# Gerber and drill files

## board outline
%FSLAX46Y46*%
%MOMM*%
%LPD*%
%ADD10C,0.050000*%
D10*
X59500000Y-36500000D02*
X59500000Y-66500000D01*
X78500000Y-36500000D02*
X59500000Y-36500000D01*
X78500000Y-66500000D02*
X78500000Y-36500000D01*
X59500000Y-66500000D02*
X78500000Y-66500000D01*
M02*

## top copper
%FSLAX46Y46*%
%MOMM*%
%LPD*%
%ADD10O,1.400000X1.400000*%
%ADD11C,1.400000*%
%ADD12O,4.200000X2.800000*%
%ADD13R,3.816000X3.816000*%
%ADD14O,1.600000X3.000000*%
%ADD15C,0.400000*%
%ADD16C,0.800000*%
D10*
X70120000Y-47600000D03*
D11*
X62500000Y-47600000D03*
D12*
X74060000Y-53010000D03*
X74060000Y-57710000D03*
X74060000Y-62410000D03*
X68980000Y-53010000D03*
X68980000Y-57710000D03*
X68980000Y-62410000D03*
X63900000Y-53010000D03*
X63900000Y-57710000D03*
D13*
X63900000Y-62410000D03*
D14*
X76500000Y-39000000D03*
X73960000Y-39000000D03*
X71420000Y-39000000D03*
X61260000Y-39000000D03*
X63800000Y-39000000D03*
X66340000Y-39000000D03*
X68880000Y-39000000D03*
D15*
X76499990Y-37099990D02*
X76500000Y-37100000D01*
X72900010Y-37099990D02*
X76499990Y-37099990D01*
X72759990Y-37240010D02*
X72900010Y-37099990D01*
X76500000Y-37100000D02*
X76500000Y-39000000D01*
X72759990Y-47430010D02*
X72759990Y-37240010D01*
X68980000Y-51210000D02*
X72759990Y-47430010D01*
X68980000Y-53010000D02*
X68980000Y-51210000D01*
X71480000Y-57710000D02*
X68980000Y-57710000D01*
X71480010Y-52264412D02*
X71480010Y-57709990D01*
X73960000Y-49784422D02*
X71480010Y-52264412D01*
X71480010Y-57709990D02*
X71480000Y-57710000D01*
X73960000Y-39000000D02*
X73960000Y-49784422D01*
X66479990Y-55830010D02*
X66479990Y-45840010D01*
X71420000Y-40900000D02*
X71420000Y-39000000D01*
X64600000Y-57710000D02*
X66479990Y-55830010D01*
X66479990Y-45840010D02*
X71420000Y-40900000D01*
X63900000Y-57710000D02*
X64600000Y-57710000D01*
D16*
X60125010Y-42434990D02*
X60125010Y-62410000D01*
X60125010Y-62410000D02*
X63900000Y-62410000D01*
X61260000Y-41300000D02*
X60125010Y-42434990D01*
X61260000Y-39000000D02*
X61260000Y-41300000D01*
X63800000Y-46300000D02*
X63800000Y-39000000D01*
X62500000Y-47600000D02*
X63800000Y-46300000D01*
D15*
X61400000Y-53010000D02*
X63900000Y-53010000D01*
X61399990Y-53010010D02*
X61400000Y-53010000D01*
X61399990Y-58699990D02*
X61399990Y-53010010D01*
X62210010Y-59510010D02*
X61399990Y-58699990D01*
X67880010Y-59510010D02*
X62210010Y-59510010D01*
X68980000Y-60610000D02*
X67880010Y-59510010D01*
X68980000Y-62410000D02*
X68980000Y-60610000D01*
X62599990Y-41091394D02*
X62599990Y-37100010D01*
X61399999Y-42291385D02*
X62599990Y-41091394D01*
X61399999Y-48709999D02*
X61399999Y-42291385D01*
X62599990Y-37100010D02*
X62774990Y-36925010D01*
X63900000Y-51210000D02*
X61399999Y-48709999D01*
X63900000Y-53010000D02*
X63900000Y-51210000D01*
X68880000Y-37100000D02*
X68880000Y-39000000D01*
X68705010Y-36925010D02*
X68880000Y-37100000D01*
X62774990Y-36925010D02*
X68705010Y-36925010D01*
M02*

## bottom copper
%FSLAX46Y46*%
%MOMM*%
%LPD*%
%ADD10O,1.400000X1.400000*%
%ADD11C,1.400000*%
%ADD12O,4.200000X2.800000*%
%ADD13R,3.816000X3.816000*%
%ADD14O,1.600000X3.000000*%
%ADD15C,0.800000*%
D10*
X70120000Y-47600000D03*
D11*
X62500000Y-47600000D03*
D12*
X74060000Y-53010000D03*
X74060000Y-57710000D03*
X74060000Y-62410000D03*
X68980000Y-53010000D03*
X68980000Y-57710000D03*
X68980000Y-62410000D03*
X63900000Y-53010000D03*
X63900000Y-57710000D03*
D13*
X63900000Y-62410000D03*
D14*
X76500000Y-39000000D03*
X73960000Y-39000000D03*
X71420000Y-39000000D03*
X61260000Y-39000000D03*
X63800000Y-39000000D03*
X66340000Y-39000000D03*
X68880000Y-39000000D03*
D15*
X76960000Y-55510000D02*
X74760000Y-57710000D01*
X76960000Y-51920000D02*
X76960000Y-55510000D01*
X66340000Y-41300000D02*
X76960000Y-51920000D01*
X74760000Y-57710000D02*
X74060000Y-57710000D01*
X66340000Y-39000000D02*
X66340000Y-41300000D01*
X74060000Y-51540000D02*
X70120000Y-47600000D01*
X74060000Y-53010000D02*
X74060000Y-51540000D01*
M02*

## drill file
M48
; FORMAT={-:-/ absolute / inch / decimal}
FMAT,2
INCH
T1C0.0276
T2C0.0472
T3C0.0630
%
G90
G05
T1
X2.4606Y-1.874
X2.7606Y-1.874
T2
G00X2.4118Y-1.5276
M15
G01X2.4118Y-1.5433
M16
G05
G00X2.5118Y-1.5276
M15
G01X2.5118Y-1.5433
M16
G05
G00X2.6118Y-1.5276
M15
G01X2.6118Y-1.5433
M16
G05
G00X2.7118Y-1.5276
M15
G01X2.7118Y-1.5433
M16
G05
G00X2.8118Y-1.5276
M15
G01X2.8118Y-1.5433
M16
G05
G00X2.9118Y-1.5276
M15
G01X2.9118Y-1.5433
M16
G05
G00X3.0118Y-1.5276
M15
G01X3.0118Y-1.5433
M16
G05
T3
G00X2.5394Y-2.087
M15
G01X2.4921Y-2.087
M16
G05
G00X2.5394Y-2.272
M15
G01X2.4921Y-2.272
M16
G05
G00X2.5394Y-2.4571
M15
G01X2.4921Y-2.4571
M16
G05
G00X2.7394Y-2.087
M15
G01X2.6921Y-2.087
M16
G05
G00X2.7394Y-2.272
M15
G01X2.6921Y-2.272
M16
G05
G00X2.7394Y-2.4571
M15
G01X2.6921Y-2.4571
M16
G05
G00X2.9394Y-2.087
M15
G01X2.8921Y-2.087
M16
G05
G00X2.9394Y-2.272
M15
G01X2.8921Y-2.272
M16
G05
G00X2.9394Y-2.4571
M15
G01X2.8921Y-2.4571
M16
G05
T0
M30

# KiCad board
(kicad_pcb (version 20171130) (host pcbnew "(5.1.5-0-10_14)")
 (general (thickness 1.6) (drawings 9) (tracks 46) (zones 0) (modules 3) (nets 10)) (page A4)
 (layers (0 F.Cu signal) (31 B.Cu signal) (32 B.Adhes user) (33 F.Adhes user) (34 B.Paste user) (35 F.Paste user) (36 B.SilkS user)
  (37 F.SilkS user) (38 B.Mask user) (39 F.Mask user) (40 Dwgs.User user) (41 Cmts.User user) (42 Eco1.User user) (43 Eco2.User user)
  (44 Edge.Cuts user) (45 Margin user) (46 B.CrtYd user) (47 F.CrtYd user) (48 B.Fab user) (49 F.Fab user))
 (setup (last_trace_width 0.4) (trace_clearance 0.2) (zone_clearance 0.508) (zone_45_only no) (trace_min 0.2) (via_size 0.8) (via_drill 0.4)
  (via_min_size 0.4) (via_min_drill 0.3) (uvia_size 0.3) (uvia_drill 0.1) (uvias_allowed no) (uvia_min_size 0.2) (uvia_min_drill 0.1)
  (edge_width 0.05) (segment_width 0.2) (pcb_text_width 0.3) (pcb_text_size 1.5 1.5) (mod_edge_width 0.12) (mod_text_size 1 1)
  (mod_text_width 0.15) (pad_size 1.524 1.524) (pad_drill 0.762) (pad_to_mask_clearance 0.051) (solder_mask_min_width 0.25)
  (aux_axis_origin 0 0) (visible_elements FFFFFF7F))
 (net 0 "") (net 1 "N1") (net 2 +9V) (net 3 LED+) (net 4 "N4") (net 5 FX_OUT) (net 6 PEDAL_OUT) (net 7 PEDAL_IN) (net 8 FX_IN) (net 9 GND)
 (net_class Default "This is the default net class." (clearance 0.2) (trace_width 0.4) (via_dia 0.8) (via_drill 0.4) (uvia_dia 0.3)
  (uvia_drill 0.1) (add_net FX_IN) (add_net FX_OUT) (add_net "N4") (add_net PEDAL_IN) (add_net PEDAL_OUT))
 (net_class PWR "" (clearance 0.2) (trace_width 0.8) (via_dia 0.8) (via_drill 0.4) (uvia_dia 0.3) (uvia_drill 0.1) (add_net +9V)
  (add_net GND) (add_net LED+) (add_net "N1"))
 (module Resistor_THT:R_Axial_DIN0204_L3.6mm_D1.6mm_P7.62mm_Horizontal (layer B.Cu) (at 62.5 47.6)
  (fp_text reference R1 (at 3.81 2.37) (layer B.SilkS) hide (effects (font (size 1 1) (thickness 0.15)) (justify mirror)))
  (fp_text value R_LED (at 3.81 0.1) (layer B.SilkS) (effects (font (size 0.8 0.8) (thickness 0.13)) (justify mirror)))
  (pad 2 thru_hole oval (at 7.62 0) (size 1.4 1.4) (drill 0.7) (layers *.Cu *.Mask) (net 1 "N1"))
  (pad 1 thru_hole circle (at 0 0) (size 1.4 1.4) (drill 0.7) (layers *.Cu *.Mask) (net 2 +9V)))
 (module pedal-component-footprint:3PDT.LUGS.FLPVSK (layer B.Cu) (at 68.98 57.71)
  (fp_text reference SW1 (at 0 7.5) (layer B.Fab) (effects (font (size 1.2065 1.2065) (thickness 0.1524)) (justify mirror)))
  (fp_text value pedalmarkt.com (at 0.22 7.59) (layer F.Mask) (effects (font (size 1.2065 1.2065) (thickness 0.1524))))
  (pad 9 thru_hole oval (at 5.08 -4.7 180) (size 4.2 2.8) (drill oval 2.8 1.6) (layers *.Cu *.Mask) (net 1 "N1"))
  (pad 8 thru_hole oval (at 5.08 0 180) (size 4.2 2.8) (drill oval 2.8 1.6) (layers *.Cu *.Mask) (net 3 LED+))
  (pad 7 thru_hole oval (at 5.08 4.7 180) (size 4.2 2.8) (drill oval 2.8 1.6) (layers *.Cu *.Mask) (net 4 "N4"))
  (pad 6 thru_hole oval (at 0 -4.7 180) (size 4.2 2.8) (drill oval 2.8 1.6) (layers *.Cu *.Mask) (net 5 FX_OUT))
  (pad 5 thru_hole oval (at 0 0 180) (size 4.2 2.8) (drill oval 2.8 1.6) (layers *.Cu *.Mask) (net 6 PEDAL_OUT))
  (pad 4 thru_hole oval (at 0 4.7 180) (size 4.2 2.8) (drill oval 2.8 1.6) (layers *.Cu *.Mask) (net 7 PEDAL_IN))
  (pad 3 thru_hole oval (at -5.08 -4.7 180) (size 4.2 2.8) (drill oval 2.8 1.6) (layers *.Cu *.Mask) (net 7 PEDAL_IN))
  (pad 2 thru_hole oval (at -5.08 0 180) (size 4.2 2.8) (drill oval 2.8 1.6) (layers *.Cu *.Mask) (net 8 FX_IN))
  (pad 1 thru_hole rect (at -5.08 4.7 180) (size 3.816 3.816) (drill oval 2.8 1.6) (layers *.Cu *.Mask) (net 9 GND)))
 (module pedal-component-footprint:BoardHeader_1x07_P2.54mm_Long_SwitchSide (layer F.Cu) (at 68.88 39)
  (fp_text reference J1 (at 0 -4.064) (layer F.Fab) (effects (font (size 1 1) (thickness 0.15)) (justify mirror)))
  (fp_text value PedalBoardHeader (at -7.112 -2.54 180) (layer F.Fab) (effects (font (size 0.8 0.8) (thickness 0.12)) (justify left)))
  (pad 7 thru_hole oval (at 7.62 0) (size 1.6 3) (drill oval 1.2 1.6) (layers *.Cu *.Mask) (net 5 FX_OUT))
  (pad 6 thru_hole oval (at 5.08 0) (size 1.6 3) (drill oval 1.2 1.6) (layers *.Cu *.Mask) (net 6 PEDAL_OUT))
  (pad 5 thru_hole oval (at 2.54 0) (size 1.6 3) (drill oval 1.2 1.6) (layers *.Cu *.Mask) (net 8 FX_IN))
  (pad 1 thru_hole oval (at -7.62 0) (size 1.6 3) (drill oval 1.2 1.6) (layers *.Cu *.Mask) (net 9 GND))
  (pad 2 thru_hole oval (at -5.08 0) (size 1.6 3) (drill oval 1.2 1.6) (layers *.Cu *.Mask) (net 2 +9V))
  (pad 3 thru_hole oval (at -2.54 0) (size 1.6 3) (drill oval 1.2 1.6) (layers *.Cu *.Mask) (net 3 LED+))
  (pad 4 thru_hole oval (at 0 0) (size 1.6 3) (drill oval 1.2 1.6) (layers *.Cu *.Mask) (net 7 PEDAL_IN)))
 (gr_line (start 59.5 36.5) (end 59.5 66.5) (layer Edge.Cuts) (width 0.05))
 (gr_line (start 78.5 36.5) (end 59.5 36.5) (layer Edge.Cuts) (width 0.05))
 (gr_line (start 78.5 66.5) (end 78.5 36.5) (layer Edge.Cuts) (width 0.05))
 (gr_line (start 59.5 66.5) (end 78.5 66.5) (layer Edge.Cuts) (width 0.05))
 (segment (start 76.49999 37.09999) (end 76.5 37.1) (width 0.4) (layer F.Cu) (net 5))
 (segment (start 72.90001 37.09999) (end 76.49999 37.09999) (width 0.4) (layer F.Cu) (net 5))
 (segment (start 72.75999 37.24001) (end 72.90001 37.09999) (width 0.4) (layer F.Cu) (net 5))
 (segment (start 76.5 37.1) (end 76.5 39) (width 0.4) (layer F.Cu) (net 5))
 (segment (start 72.75999 47.43001) (end 72.75999 37.24001) (width 0.4) (layer F.Cu) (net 5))
 (segment (start 68.98 51.21) (end 72.75999 47.43001) (width 0.4) (layer F.Cu) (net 5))
 (segment (start 68.98 53.01) (end 68.98 51.21) (width 0.4) (layer F.Cu) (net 5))
 (segment (start 71.48 57.71) (end 68.98 57.71) (width 0.4) (layer F.Cu) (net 6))
 (segment (start 71.48001 52.264412) (end 71.48001 57.70999) (width 0.4) (layer F.Cu) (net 6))
 (segment (start 73.96 49.784422) (end 71.48001 52.264412) (width 0.4) (layer F.Cu) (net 6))
 (segment (start 71.48001 57.70999) (end 71.48 57.71) (width 0.4) (layer F.Cu) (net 6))
 (segment (start 73.96 39) (end 73.96 49.784422) (width 0.4) (layer F.Cu) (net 6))
 (segment (start 66.47999 55.83001) (end 66.47999 45.84001) (width 0.4) (layer F.Cu) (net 8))
 (segment (start 71.42 40.9) (end 71.42 39) (width 0.4) (layer F.Cu) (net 8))
 (segment (start 64.6 57.71) (end 66.47999 55.83001) (width 0.4) (layer F.Cu) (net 8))
 (segment (start 66.47999 45.84001) (end 71.42 40.9) (width 0.4) (layer F.Cu) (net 8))
 (segment (start 63.9 57.71) (end 64.6 57.71) (width 0.4) (layer F.Cu) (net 8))
 (segment (start 60.12501 42.43499) (end 60.12501 62.41) (width 0.8) (layer F.Cu) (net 9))
 (segment (start 60.12501 62.41) (end 63.9 62.41) (width 0.8) (layer F.Cu) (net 9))
 (segment (start 61.26 41.3) (end 60.12501 42.43499) (width 0.8) (layer F.Cu) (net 9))
 (segment (start 61.26 39) (end 61.26 41.3) (width 0.8) (layer F.Cu) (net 9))
 (segment (start 63.8 46.3) (end 63.8 39) (width 0.8) (layer F.Cu) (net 2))
 (segment (start 62.5 47.6) (end 63.8 46.3) (width 0.8) (layer F.Cu) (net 2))
 (segment (start 76.96 55.51) (end 74.76 57.71) (width 0.8) (layer B.Cu) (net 3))
 (segment (start 76.96 51.92) (end 76.96 55.51) (width 0.8) (layer B.Cu) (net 3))
 (segment (start 66.34 41.3) (end 76.96 51.92) (width 0.8) (layer B.Cu) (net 3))
 (segment (start 74.76 57.71) (end 74.06 57.71) (width 0.8) (layer B.Cu) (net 3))
 (segment (start 66.34 39) (end 66.34 41.3) (width 0.8) (layer B.Cu) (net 3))
 (segment (start 61.4 53.01) (end 63.9 53.01) (width 0.4) (layer F.Cu) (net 7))
 (segment (start 61.39999 53.01001) (end 61.4 53.01) (width 0.4) (layer F.Cu) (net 7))
 (segment (start 61.39999 58.69999) (end 61.39999 53.01001) (width 0.4) (layer F.Cu) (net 7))
 (segment (start 62.21001 59.51001) (end 61.39999 58.69999) (width 0.4) (layer F.Cu) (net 7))
 (segment (start 67.88001 59.51001) (end 62.21001 59.51001) (width 0.4) (layer F.Cu) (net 7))
 (segment (start 68.98 60.61) (end 67.88001 59.51001) (width 0.4) (layer F.Cu) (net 7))
 (segment (start 68.98 62.41) (end 68.98 60.61) (width 0.4) (layer F.Cu) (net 7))
 (segment (start 62.59999 41.091394) (end 62.59999 37.10001) (width 0.4) (layer F.Cu) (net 7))
 (segment (start 61.399999 42.291385) (end 62.59999 41.091394) (width 0.4) (layer F.Cu) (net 7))
 (segment (start 61.399999 48.709999) (end 61.399999 42.291385) (width 0.4) (layer F.Cu) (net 7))
 (segment (start 62.59999 37.10001) (end 62.77499 36.92501) (width 0.4) (layer F.Cu) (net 7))
 (segment (start 63.9 51.21) (end 61.399999 48.709999) (width 0.4) (layer F.Cu) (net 7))
 (segment (start 63.9 53.01) (end 63.9 51.21) (width 0.4) (layer F.Cu) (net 7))
 (segment (start 68.88 37.1) (end 68.88 39) (width 0.4) (layer F.Cu) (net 7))
 (segment (start 68.70501 36.92501) (end 68.88 37.1) (width 0.4) (layer F.Cu) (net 7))
 (segment (start 62.77499 36.92501) (end 68.70501 36.92501) (width 0.4) (layer F.Cu) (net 7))
 (segment (start 74.06 51.54) (end 70.12 47.6) (width 0.8) (layer B.Cu) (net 1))
 (segment (start 74.06 53.01) (end 74.06 51.54) (width 0.8) (layer B.Cu) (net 1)))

